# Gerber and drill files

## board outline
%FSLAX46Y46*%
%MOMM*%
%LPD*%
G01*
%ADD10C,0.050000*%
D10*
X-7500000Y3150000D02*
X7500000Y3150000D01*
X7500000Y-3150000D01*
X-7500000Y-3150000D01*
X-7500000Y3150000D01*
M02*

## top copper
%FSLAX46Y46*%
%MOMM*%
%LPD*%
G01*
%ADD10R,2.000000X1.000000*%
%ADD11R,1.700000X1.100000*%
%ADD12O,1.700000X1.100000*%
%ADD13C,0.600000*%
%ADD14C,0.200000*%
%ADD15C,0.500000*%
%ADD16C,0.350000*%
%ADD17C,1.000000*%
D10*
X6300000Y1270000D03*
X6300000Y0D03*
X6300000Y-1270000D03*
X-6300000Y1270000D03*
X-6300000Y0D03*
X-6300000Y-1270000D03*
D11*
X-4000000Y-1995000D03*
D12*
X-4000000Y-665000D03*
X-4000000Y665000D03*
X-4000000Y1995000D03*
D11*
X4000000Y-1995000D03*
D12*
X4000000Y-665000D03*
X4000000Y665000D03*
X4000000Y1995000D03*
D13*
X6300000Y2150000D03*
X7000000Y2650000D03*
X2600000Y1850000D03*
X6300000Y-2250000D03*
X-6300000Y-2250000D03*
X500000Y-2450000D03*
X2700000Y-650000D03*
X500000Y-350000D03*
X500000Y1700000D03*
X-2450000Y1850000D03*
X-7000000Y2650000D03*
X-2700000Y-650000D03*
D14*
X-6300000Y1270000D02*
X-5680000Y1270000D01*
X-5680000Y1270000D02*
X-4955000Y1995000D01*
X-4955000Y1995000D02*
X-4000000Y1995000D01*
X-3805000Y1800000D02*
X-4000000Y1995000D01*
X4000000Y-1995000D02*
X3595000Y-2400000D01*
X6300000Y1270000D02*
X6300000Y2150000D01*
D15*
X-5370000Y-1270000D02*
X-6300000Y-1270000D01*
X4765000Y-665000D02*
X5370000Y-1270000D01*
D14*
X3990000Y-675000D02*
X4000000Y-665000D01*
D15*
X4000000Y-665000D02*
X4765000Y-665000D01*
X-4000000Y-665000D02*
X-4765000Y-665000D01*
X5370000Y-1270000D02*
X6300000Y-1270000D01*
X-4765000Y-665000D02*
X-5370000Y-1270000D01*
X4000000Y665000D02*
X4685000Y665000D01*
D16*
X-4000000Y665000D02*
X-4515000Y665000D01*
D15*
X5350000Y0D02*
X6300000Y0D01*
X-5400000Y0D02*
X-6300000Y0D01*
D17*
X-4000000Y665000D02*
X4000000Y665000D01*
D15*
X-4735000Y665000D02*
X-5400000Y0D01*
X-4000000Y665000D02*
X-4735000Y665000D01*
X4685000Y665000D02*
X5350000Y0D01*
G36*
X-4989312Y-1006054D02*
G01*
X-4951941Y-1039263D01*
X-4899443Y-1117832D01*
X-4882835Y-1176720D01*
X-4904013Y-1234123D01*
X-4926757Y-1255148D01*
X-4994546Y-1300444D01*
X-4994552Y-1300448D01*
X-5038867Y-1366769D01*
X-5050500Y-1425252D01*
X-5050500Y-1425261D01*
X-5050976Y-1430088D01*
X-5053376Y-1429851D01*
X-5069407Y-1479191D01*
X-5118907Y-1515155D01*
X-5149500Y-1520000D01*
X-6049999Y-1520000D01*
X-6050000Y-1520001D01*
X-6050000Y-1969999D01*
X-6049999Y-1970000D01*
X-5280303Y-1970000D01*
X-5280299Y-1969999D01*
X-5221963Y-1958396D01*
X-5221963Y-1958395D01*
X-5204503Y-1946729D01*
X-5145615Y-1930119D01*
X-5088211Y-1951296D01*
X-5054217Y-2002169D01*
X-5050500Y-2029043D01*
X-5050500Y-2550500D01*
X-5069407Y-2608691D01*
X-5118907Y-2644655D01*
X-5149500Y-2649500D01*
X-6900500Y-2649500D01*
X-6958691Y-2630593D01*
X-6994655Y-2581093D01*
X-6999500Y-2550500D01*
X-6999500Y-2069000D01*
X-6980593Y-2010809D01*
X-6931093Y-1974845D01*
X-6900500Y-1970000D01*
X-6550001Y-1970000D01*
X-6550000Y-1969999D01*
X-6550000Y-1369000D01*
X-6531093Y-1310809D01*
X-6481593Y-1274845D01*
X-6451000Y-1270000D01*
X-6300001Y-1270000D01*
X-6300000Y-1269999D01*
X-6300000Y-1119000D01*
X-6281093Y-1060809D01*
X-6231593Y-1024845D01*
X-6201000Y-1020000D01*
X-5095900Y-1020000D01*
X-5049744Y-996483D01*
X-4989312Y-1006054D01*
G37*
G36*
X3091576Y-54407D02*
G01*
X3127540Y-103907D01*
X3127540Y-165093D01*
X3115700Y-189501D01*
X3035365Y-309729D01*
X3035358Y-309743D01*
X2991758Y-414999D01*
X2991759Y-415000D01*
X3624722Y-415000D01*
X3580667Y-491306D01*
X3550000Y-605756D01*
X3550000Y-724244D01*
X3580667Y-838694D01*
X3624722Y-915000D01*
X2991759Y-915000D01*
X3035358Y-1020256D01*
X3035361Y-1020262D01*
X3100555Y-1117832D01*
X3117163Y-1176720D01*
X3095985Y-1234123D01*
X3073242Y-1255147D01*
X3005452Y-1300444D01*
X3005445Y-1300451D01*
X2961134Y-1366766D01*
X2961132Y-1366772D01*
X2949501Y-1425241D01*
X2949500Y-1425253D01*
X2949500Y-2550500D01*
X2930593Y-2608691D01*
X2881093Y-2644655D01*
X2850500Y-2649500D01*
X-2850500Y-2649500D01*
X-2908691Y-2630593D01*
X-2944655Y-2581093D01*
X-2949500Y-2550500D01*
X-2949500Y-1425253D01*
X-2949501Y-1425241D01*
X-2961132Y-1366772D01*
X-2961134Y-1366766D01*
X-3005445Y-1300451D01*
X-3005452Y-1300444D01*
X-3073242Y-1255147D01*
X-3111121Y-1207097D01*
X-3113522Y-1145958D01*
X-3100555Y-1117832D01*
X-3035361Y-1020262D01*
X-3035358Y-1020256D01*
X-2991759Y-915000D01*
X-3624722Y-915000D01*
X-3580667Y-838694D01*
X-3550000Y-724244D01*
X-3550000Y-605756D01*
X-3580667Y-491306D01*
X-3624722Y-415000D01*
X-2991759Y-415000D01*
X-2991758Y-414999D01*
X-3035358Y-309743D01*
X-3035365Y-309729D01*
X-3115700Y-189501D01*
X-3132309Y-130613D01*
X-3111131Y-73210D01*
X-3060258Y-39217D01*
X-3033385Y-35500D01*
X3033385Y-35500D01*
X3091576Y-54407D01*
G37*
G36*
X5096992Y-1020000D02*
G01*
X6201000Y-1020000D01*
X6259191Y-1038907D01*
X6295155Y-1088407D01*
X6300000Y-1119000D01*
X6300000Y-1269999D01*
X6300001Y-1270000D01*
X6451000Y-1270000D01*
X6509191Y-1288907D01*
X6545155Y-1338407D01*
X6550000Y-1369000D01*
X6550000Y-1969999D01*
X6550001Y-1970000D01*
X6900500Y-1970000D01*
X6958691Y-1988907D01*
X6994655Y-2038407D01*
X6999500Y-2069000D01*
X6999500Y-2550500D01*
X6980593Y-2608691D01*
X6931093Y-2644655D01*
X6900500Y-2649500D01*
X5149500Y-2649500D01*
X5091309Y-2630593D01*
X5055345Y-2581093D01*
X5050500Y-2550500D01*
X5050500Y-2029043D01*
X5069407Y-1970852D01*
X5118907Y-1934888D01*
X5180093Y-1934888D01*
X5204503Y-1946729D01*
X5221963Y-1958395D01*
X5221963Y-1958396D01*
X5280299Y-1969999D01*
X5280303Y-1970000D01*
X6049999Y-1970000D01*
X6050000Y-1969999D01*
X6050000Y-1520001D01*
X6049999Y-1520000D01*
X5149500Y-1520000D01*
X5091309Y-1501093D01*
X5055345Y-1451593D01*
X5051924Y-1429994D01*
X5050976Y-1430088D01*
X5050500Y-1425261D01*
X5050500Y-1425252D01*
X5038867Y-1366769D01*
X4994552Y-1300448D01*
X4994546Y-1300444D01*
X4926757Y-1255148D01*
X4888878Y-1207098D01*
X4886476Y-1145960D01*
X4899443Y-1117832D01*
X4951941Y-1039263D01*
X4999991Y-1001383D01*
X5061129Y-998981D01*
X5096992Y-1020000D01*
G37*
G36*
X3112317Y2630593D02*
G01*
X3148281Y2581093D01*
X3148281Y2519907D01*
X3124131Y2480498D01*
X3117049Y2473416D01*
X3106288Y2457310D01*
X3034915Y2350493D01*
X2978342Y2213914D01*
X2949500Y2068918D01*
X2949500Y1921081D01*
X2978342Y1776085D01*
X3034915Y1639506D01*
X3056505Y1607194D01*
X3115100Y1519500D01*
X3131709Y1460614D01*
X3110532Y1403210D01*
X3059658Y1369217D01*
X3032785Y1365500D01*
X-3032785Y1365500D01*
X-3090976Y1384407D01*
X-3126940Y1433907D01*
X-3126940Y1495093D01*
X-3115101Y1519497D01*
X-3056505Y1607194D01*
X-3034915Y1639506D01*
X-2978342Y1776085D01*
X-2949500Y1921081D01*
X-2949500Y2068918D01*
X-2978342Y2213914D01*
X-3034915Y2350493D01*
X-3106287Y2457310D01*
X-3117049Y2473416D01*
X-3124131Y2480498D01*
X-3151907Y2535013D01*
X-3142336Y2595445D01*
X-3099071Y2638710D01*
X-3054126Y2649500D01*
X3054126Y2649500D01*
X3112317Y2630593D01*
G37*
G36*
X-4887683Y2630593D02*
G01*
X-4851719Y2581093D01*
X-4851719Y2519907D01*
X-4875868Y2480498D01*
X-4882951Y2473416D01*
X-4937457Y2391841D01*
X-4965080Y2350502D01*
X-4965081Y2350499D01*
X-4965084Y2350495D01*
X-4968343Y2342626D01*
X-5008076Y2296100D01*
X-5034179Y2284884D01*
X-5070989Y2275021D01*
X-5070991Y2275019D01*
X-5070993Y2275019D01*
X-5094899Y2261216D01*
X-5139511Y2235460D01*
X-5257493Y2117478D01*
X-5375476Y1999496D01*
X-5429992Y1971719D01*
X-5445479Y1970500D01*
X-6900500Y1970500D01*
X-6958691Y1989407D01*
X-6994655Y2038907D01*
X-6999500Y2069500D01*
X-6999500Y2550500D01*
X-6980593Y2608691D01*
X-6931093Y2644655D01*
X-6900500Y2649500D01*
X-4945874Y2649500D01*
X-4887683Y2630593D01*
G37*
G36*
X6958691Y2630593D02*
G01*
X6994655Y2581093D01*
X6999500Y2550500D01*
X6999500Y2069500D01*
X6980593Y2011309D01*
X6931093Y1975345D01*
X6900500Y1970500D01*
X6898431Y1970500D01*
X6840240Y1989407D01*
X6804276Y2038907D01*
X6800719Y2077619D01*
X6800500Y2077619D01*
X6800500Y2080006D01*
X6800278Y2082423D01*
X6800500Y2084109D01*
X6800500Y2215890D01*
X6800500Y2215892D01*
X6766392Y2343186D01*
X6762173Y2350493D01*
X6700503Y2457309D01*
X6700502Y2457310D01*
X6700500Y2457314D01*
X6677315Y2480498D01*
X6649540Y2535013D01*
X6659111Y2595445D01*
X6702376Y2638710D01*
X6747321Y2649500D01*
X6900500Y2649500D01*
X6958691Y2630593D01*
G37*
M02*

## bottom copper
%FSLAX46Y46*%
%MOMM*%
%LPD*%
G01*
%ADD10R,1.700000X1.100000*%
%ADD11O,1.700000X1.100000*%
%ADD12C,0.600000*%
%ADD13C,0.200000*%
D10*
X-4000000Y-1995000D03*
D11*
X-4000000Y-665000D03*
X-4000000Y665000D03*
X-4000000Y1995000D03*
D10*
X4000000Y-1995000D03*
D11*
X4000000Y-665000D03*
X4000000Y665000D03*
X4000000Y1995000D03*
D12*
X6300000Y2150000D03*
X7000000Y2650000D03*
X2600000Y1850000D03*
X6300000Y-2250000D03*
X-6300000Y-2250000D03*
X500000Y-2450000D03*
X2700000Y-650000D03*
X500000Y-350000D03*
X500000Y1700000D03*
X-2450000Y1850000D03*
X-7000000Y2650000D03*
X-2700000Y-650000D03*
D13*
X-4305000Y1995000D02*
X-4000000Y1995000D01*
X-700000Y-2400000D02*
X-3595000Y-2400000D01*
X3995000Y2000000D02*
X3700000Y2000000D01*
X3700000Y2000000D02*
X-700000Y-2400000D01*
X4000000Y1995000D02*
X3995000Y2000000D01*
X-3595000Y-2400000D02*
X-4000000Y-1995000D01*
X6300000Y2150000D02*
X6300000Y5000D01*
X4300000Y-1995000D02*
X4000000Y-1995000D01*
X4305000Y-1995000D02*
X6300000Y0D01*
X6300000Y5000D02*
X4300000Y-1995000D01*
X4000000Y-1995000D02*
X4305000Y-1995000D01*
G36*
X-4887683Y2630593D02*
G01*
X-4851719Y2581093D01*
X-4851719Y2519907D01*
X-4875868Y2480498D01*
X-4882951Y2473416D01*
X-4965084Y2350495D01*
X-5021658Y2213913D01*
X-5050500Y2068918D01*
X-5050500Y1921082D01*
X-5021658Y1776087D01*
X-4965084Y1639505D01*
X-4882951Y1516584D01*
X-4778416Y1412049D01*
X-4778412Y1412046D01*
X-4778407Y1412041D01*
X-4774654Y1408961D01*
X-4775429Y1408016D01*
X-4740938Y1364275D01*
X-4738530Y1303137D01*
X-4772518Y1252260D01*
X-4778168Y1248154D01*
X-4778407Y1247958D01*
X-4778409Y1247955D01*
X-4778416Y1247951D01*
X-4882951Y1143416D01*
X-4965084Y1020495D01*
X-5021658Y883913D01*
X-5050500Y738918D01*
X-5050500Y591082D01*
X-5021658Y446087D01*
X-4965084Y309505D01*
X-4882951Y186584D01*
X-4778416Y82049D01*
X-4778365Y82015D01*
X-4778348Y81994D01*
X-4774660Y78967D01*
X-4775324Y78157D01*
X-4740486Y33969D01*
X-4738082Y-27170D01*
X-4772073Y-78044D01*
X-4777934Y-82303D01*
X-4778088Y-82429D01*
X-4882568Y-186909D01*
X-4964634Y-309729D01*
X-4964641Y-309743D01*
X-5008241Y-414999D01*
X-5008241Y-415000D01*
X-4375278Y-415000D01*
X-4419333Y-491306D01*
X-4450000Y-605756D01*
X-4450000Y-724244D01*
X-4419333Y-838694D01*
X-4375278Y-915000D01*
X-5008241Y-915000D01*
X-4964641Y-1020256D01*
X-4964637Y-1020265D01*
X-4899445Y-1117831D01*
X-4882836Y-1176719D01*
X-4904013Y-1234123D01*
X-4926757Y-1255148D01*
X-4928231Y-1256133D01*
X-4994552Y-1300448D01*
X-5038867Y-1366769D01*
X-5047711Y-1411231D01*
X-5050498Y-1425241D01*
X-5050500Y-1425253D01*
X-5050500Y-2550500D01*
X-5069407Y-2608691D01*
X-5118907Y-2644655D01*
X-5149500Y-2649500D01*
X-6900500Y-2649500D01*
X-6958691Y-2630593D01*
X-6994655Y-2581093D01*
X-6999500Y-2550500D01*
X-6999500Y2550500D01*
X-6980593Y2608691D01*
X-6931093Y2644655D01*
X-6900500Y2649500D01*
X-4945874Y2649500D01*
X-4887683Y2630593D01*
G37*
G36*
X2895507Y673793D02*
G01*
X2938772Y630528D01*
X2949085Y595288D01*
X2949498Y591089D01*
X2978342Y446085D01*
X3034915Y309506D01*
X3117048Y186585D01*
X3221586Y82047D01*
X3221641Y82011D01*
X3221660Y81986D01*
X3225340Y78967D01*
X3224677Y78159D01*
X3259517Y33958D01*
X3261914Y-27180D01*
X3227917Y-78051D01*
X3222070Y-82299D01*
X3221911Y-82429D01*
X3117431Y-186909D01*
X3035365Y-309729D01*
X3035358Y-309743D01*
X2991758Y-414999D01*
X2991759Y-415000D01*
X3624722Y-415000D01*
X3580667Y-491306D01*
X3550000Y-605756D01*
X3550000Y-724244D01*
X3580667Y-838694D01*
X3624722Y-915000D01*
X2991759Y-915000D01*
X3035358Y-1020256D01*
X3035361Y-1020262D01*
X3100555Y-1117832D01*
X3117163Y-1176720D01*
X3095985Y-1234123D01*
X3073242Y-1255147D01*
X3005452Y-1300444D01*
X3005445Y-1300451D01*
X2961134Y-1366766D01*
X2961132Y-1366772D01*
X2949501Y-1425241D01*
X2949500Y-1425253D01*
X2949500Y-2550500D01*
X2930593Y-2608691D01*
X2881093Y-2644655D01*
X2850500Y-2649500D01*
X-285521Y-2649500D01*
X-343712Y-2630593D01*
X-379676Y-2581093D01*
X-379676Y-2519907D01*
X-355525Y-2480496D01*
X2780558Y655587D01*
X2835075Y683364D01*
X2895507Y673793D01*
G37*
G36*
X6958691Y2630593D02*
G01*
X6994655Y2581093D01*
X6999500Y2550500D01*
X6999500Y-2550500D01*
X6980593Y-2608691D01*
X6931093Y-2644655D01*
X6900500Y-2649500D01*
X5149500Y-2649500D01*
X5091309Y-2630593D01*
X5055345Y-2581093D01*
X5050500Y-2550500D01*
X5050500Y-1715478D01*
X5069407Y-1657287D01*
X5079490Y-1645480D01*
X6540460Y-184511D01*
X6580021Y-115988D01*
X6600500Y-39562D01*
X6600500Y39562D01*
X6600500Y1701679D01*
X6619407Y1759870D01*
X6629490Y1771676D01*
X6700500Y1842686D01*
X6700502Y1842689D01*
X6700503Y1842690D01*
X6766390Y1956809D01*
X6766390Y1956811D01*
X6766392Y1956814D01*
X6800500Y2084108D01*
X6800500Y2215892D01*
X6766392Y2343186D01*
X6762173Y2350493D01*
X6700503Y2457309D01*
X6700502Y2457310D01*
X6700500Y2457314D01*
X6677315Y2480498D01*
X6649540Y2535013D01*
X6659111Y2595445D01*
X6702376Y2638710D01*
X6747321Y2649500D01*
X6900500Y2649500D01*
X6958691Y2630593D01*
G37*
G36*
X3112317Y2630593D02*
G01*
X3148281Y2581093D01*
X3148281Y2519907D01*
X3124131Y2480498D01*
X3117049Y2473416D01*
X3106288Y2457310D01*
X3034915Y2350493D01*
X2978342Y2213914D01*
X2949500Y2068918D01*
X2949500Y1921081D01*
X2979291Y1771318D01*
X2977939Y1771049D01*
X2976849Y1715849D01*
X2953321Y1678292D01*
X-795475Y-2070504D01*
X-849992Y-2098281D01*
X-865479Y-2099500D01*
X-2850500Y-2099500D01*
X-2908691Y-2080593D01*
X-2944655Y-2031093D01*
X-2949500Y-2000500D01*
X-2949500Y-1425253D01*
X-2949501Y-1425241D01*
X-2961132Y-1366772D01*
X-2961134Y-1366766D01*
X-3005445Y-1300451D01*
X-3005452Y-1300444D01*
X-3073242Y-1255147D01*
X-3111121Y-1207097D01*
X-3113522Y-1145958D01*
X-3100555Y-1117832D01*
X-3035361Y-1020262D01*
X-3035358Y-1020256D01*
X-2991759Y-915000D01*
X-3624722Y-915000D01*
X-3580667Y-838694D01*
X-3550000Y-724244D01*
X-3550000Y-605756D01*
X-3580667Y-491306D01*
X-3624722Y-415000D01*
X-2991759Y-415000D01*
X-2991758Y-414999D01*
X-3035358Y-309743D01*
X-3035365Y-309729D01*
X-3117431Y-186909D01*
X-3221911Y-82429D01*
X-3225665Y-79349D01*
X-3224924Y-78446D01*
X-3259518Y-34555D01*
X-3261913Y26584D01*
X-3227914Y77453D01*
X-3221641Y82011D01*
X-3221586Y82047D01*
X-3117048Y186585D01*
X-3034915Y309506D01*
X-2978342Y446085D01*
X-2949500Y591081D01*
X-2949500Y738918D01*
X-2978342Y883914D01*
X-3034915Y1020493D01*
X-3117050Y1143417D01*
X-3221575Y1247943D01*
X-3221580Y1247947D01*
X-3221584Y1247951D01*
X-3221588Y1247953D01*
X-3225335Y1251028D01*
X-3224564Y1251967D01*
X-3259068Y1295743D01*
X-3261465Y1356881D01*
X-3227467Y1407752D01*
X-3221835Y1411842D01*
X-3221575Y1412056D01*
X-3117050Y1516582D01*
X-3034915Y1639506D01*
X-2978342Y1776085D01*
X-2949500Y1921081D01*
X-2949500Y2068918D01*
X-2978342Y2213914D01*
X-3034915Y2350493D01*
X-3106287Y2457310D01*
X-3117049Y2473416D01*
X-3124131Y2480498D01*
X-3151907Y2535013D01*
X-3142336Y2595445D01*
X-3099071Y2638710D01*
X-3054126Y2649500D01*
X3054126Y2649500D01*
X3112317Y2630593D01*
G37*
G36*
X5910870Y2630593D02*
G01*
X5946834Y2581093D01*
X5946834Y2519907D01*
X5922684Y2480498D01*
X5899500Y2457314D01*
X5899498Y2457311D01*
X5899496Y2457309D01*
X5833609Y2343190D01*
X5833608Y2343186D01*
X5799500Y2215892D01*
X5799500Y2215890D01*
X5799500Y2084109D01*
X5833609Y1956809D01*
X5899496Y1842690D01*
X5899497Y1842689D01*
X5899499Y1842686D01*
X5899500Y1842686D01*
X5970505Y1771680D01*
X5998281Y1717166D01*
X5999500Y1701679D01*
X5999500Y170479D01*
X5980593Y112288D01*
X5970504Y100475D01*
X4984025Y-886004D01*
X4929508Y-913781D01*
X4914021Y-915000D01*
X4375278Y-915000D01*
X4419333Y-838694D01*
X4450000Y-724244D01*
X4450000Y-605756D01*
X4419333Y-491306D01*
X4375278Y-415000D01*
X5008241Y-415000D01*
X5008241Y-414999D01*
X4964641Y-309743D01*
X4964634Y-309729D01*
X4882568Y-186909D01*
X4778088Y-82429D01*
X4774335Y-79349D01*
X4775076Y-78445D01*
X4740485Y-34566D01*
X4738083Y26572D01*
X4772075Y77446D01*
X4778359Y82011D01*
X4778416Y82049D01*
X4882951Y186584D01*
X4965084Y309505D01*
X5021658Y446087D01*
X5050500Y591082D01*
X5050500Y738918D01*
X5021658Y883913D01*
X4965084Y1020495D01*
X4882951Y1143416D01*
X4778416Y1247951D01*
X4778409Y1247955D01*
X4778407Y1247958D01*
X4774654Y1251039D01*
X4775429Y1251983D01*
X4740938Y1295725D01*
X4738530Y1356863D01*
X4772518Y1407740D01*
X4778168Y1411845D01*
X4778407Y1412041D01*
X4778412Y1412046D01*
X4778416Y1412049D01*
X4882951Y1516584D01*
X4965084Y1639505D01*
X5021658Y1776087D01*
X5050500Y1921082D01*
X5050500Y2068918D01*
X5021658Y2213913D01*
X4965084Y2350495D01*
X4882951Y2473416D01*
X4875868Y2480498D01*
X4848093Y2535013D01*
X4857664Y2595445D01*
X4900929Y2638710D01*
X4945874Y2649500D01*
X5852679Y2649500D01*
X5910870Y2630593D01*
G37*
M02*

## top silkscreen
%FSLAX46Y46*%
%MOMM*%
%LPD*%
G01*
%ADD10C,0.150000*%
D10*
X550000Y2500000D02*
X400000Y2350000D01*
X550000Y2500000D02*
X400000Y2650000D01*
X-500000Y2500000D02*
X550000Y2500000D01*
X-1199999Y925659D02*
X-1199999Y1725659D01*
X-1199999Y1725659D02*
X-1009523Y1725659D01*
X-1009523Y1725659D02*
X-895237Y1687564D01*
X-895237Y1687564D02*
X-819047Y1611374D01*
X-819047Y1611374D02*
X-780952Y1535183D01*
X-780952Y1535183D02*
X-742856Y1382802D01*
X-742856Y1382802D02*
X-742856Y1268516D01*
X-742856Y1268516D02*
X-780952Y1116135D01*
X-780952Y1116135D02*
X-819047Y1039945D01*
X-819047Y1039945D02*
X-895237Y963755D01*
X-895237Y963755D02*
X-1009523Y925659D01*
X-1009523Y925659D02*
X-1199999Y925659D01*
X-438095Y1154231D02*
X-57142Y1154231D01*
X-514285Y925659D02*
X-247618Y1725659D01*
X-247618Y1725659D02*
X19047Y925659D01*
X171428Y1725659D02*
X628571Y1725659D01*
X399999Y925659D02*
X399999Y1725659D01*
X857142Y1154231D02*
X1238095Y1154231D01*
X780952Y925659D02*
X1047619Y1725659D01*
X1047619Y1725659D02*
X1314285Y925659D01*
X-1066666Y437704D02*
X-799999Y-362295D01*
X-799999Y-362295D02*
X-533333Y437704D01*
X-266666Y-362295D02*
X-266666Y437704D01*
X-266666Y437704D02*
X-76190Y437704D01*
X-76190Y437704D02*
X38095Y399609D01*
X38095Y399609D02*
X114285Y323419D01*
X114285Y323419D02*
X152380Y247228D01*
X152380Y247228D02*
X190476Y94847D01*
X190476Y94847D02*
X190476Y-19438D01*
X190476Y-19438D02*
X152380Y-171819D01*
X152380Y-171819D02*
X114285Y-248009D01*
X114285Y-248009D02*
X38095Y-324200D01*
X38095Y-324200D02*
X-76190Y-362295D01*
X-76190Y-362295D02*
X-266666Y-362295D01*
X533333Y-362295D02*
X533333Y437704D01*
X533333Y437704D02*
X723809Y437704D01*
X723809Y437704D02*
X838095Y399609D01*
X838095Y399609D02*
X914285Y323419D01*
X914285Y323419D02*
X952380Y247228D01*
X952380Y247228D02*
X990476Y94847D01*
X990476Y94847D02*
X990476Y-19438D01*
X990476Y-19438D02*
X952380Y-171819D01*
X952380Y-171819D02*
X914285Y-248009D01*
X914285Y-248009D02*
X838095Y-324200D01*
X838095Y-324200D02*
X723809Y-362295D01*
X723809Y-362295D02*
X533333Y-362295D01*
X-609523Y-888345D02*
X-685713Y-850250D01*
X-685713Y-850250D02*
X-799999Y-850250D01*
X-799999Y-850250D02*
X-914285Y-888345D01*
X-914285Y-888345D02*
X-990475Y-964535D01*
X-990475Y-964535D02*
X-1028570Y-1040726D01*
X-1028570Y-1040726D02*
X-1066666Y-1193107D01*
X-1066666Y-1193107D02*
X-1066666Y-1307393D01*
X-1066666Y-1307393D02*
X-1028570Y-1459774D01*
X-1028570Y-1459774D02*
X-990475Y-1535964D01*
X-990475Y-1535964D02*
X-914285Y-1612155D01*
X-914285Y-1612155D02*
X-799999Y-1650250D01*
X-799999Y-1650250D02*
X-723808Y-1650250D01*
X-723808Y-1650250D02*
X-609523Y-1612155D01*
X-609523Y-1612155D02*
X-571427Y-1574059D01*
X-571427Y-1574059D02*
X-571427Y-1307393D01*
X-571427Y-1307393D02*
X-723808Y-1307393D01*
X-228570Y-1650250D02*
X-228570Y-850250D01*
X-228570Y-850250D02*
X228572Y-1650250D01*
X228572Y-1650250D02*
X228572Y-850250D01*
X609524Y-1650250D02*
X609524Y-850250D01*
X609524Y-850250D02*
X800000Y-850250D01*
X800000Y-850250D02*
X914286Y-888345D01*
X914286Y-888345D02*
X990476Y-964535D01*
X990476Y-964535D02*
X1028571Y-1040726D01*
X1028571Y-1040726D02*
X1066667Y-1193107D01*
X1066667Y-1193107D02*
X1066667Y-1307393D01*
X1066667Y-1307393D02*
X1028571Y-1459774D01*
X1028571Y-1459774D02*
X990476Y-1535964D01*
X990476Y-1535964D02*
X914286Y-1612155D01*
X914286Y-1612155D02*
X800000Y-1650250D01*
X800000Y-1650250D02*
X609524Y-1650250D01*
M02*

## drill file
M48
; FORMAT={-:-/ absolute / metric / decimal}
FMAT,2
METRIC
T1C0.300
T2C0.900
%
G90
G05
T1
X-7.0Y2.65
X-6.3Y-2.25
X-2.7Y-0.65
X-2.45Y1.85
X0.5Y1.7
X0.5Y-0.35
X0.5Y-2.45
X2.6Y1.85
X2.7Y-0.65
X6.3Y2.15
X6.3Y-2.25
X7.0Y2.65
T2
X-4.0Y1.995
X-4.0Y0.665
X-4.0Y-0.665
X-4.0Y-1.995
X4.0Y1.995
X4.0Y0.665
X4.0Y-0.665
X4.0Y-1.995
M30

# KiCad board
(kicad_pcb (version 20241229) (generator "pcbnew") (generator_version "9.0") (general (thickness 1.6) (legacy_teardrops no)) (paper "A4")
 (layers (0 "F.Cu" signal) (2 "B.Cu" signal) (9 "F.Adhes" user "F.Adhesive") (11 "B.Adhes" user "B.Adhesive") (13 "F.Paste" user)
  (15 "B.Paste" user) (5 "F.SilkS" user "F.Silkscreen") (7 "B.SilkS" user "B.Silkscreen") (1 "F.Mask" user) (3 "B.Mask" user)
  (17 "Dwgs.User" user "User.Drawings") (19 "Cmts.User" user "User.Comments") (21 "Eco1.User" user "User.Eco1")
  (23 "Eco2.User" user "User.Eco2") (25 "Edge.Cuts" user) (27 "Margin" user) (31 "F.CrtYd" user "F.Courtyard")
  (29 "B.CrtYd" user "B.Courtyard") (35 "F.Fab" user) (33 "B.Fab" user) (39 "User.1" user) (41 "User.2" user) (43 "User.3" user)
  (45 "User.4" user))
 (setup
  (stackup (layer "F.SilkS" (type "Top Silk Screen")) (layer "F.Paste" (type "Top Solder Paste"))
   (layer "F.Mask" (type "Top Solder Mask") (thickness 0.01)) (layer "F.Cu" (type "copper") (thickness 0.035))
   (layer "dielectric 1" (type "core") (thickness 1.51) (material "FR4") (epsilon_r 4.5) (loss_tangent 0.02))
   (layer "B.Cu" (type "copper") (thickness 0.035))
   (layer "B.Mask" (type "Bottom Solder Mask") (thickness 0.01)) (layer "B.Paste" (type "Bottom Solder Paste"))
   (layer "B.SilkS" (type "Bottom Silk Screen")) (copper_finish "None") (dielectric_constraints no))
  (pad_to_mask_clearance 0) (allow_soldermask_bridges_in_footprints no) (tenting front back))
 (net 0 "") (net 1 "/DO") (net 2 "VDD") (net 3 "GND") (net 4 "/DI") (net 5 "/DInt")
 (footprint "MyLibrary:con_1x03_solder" (layer "F.Cu") (at 6.3 0)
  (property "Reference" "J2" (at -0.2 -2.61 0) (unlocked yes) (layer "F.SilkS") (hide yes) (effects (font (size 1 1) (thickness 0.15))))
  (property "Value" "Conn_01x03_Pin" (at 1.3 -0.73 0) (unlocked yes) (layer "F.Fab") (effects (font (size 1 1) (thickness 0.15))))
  (pad "1" smd rect (at 0 -1.27) (size 2 1) (layers "F.Cu" "F.Mask" "F.Paste") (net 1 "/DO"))
  (pad "2" smd rect (at 0 0) (size 2 1) (layers "F.Cu" "F.Mask" "F.Paste") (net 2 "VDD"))
  (pad "3" smd rect (at 0 1.27) (size 2 1) (layers "F.Cu" "F.Mask" "F.Paste") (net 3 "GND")))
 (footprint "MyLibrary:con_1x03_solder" (layer "F.Cu") (at -6.3 0)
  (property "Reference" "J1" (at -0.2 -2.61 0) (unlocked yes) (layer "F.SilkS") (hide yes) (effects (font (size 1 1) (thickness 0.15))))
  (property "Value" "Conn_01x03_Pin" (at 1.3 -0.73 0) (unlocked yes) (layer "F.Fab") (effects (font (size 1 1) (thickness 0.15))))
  (pad "1" smd rect (at 0 -1.27) (size 2 1) (layers "F.Cu" "F.Mask" "F.Paste") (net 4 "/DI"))
  (pad "2" smd rect (at 0 0) (size 2 1) (layers "F.Cu" "F.Mask" "F.Paste") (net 2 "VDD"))
  (pad "3" smd rect (at 0 1.27) (size 2 1) (layers "F.Cu" "F.Mask" "F.Paste") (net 3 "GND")))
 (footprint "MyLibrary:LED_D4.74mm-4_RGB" (layer "B.Cu") (at -4 0 90)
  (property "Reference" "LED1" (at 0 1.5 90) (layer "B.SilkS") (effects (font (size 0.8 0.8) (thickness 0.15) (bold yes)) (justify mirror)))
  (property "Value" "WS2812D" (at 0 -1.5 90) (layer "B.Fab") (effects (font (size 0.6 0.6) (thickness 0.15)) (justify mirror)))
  (pad "1" thru_hole rect (at -1.995 0 90) (size 1.1 1.7) (drill 0.9) (layers "*.Cu" "*.Mask") (remove_unused_layers no) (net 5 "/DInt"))
  (pad "2" thru_hole oval (at -0.665 0 90) (size 1.1 1.7) (drill 0.9) (layers "*.Cu" "*.Mask") (remove_unused_layers no) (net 3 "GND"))
  (pad "3" thru_hole oval (at 0.665 0 90) (size 1.1 1.7) (drill 0.9) (layers "*.Cu" "*.Mask") (remove_unused_layers no) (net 2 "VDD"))
  (pad "4" thru_hole oval (at 1.995 0 90) (size 1.1 1.7) (drill 0.9) (layers "*.Cu" "*.Mask") (remove_unused_layers no) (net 4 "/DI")))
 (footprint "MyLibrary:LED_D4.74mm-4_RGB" (layer "B.Cu") (at 4 0 90)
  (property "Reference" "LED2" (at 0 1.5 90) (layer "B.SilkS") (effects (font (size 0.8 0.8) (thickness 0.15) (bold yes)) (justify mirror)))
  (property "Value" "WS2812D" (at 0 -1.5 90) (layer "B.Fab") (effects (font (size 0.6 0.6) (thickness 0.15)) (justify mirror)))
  (pad "1" thru_hole rect (at -1.995 0 90) (size 1.1 1.7) (drill 0.9) (layers "*.Cu" "*.Mask") (remove_unused_layers no) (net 1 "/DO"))
  (pad "2" thru_hole oval (at -0.665 0 90) (size 1.1 1.7) (drill 0.9) (layers "*.Cu" "*.Mask") (remove_unused_layers no) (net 3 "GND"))
  (pad "3" thru_hole oval (at 0.665 0 90) (size 1.1 1.7) (drill 0.9) (layers "*.Cu" "*.Mask") (remove_unused_layers no) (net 2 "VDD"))
  (pad "4" thru_hole oval (at 1.995 0 90) (size 1.1 1.7) (drill 0.9) (layers "*.Cu" "*.Mask") (remove_unused_layers no) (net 5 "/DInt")))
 (gr_line (start 0.55 -2.5) (end 0.4 -2.35) (stroke (width 0.15) (type default)) (layer "F.SilkS"))
 (gr_line (start 0.55 -2.5) (end 0.4 -2.65) (stroke (width 0.15) (type default)) (layer "F.SilkS"))
 (gr_line (start -0.5 -2.5) (end 0.55 -2.5) (stroke (width 0.15) (type solid)) (layer "F.SilkS"))
 (gr_rect (start -7.5 -3.15) (end 7.5 3.15) (stroke (width 0.05) (type solid)) (fill no) (layer "Edge.Cuts"))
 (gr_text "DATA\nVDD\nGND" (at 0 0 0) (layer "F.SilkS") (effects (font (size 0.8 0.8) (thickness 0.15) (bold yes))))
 (segment (start -6.3 -1.27) (end -5.68 -1.27) (width 0.2) (layer "F.Cu") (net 4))
 (segment (start -5.68 -1.27) (end -4.955 -1.995) (width 0.2) (layer "F.Cu") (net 4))
 (segment (start -4.955 -1.995) (end -4 -1.995) (width 0.2) (layer "F.Cu") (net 4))
 (segment (start -3.805 -1.8) (end -4 -1.995) (width 0.2) (layer "F.Cu") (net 4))
 (segment (start -4.305 -1.995) (end -4 -1.995) (width 0.2) (layer "B.Cu") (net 4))
 (segment (start -0.7 2.4) (end -3.595 2.4) (width 0.2) (layer "B.Cu") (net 5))
 (segment (start 3.995 -2) (end 3.7 -2) (width 0.2) (layer "B.Cu") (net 5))
 (segment (start 3.7 -2) (end -0.7 2.4) (width 0.2) (layer "B.Cu") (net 5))
 (segment (start 4 -1.995) (end 3.995 -2) (width 0.2) (layer "B.Cu") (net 5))
 (segment (start -3.595 2.4) (end -4 1.995) (width 0.2) (layer "B.Cu") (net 5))
 (segment (start 4 1.995) (end 3.595 2.4) (width 0.2) (layer "F.Cu") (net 1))
 (segment (start 6.3 -1.27) (end 6.3 -2.15) (width 0.2) (layer "F.Cu") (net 1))
 (via (at 6.3 -2.15) (size 0.6) (drill 0.3) (layers "F.Cu" "B.Cu") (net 1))
 (segment (start 6.3 -2.15) (end 6.3 -0.005) (width 0.2) (layer "B.Cu") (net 1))
 (segment (start 4.3 1.995) (end 4 1.995) (width 0.2) (layer "B.Cu") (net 1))
 (segment (start 4.305 1.995) (end 6.3 0) (width 0.2) (layer "B.Cu") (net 1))
 (segment (start 6.3 -0.005) (end 4.3 1.995) (width 0.2) (layer "B.Cu") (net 1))
 (segment (start 4 1.995) (end 4.305 1.995) (width 0.2) (layer "B.Cu") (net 1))
 (segment (start -5.37 1.27) (end -6.3 1.27) (width 0.5) (layer "F.Cu") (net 3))
 (segment (start 4.765 0.665) (end 5.37 1.27) (width 0.5) (layer "F.Cu") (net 3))
 (segment (start 3.99 0.675) (end 4 0.665) (width 0.2) (layer "F.Cu") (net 3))
 (segment (start 4 0.665) (end 4.765 0.665) (width 0.5) (layer "F.Cu") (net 3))
 (segment (start -4 0.665) (end -4.765 0.665) (width 0.5) (layer "F.Cu") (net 3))
 (segment (start 5.37 1.27) (end 6.3 1.27) (width 0.5) (layer "F.Cu") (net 3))
 (segment (start -4.765 0.665) (end -5.37 1.27) (width 0.5) (layer "F.Cu") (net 3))
 (via (at 7 -2.65) (size 0.6) (drill 0.3) (layers "F.Cu" "B.Cu") (free yes) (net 3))
 (via (at 2.6 -1.85) (size 0.6) (drill 0.3) (layers "F.Cu" "B.Cu") (free yes) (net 3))
 (via (at 6.3 2.25) (size 0.6) (drill 0.3) (layers "F.Cu" "B.Cu") (free yes) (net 3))
 (via (at -6.3 2.25) (size 0.6) (drill 0.3) (layers "F.Cu" "B.Cu") (free yes) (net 3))
 (via (at 0.5 2.45) (size 0.6) (drill 0.3) (layers "F.Cu" "B.Cu") (free yes) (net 3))
 (via (at 2.7 0.65) (size 0.6) (drill 0.3) (layers "F.Cu" "B.Cu") (free yes) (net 3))
 (via (at 0.5 0.35) (size 0.6) (drill 0.3) (layers "F.Cu" "B.Cu") (free yes) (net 3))
 (via (at 0.5 -1.7) (size 0.6) (drill 0.3) (layers "F.Cu" "B.Cu") (free yes) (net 3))
 (via (at -2.45 -1.85) (size 0.6) (drill 0.3) (layers "F.Cu" "B.Cu") (free yes) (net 3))
 (via (at -7 -2.65) (size 0.6) (drill 0.3) (layers "F.Cu" "B.Cu") (free yes) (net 3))
 (via (at -2.7 0.65) (size 0.6) (drill 0.3) (layers "F.Cu" "B.Cu") (free yes) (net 3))
 (segment (start 4 -0.665) (end 4.685 -0.665) (width 0.5) (layer "F.Cu") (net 2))
 (segment (start -4 -0.665) (end -4.515 -0.665) (width 0.35) (layer "F.Cu") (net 2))
 (segment (start 5.35 0) (end 6.3 0) (width 0.5) (layer "F.Cu") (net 2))
 (segment (start -5.4 0) (end -6.3 0) (width 0.5) (layer "F.Cu") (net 2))
 (segment (start -4 -0.665) (end 4 -0.665) (width 1) (layer "F.Cu") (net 2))
 (segment (start -4.735 -0.665) (end -5.4 0) (width 0.5) (layer "F.Cu") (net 2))
 (segment (start -4 -0.665) (end -4.735 -0.665) (width 0.5) (layer "F.Cu") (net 2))
 (segment (start 4.685 -0.665) (end 5.35 0) (width 0.5) (layer "F.Cu") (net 2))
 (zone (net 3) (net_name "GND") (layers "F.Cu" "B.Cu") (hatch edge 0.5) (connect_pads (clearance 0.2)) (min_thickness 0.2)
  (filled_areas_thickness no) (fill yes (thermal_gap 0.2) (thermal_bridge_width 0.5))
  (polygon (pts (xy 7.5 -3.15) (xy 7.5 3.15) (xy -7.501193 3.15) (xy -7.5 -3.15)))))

